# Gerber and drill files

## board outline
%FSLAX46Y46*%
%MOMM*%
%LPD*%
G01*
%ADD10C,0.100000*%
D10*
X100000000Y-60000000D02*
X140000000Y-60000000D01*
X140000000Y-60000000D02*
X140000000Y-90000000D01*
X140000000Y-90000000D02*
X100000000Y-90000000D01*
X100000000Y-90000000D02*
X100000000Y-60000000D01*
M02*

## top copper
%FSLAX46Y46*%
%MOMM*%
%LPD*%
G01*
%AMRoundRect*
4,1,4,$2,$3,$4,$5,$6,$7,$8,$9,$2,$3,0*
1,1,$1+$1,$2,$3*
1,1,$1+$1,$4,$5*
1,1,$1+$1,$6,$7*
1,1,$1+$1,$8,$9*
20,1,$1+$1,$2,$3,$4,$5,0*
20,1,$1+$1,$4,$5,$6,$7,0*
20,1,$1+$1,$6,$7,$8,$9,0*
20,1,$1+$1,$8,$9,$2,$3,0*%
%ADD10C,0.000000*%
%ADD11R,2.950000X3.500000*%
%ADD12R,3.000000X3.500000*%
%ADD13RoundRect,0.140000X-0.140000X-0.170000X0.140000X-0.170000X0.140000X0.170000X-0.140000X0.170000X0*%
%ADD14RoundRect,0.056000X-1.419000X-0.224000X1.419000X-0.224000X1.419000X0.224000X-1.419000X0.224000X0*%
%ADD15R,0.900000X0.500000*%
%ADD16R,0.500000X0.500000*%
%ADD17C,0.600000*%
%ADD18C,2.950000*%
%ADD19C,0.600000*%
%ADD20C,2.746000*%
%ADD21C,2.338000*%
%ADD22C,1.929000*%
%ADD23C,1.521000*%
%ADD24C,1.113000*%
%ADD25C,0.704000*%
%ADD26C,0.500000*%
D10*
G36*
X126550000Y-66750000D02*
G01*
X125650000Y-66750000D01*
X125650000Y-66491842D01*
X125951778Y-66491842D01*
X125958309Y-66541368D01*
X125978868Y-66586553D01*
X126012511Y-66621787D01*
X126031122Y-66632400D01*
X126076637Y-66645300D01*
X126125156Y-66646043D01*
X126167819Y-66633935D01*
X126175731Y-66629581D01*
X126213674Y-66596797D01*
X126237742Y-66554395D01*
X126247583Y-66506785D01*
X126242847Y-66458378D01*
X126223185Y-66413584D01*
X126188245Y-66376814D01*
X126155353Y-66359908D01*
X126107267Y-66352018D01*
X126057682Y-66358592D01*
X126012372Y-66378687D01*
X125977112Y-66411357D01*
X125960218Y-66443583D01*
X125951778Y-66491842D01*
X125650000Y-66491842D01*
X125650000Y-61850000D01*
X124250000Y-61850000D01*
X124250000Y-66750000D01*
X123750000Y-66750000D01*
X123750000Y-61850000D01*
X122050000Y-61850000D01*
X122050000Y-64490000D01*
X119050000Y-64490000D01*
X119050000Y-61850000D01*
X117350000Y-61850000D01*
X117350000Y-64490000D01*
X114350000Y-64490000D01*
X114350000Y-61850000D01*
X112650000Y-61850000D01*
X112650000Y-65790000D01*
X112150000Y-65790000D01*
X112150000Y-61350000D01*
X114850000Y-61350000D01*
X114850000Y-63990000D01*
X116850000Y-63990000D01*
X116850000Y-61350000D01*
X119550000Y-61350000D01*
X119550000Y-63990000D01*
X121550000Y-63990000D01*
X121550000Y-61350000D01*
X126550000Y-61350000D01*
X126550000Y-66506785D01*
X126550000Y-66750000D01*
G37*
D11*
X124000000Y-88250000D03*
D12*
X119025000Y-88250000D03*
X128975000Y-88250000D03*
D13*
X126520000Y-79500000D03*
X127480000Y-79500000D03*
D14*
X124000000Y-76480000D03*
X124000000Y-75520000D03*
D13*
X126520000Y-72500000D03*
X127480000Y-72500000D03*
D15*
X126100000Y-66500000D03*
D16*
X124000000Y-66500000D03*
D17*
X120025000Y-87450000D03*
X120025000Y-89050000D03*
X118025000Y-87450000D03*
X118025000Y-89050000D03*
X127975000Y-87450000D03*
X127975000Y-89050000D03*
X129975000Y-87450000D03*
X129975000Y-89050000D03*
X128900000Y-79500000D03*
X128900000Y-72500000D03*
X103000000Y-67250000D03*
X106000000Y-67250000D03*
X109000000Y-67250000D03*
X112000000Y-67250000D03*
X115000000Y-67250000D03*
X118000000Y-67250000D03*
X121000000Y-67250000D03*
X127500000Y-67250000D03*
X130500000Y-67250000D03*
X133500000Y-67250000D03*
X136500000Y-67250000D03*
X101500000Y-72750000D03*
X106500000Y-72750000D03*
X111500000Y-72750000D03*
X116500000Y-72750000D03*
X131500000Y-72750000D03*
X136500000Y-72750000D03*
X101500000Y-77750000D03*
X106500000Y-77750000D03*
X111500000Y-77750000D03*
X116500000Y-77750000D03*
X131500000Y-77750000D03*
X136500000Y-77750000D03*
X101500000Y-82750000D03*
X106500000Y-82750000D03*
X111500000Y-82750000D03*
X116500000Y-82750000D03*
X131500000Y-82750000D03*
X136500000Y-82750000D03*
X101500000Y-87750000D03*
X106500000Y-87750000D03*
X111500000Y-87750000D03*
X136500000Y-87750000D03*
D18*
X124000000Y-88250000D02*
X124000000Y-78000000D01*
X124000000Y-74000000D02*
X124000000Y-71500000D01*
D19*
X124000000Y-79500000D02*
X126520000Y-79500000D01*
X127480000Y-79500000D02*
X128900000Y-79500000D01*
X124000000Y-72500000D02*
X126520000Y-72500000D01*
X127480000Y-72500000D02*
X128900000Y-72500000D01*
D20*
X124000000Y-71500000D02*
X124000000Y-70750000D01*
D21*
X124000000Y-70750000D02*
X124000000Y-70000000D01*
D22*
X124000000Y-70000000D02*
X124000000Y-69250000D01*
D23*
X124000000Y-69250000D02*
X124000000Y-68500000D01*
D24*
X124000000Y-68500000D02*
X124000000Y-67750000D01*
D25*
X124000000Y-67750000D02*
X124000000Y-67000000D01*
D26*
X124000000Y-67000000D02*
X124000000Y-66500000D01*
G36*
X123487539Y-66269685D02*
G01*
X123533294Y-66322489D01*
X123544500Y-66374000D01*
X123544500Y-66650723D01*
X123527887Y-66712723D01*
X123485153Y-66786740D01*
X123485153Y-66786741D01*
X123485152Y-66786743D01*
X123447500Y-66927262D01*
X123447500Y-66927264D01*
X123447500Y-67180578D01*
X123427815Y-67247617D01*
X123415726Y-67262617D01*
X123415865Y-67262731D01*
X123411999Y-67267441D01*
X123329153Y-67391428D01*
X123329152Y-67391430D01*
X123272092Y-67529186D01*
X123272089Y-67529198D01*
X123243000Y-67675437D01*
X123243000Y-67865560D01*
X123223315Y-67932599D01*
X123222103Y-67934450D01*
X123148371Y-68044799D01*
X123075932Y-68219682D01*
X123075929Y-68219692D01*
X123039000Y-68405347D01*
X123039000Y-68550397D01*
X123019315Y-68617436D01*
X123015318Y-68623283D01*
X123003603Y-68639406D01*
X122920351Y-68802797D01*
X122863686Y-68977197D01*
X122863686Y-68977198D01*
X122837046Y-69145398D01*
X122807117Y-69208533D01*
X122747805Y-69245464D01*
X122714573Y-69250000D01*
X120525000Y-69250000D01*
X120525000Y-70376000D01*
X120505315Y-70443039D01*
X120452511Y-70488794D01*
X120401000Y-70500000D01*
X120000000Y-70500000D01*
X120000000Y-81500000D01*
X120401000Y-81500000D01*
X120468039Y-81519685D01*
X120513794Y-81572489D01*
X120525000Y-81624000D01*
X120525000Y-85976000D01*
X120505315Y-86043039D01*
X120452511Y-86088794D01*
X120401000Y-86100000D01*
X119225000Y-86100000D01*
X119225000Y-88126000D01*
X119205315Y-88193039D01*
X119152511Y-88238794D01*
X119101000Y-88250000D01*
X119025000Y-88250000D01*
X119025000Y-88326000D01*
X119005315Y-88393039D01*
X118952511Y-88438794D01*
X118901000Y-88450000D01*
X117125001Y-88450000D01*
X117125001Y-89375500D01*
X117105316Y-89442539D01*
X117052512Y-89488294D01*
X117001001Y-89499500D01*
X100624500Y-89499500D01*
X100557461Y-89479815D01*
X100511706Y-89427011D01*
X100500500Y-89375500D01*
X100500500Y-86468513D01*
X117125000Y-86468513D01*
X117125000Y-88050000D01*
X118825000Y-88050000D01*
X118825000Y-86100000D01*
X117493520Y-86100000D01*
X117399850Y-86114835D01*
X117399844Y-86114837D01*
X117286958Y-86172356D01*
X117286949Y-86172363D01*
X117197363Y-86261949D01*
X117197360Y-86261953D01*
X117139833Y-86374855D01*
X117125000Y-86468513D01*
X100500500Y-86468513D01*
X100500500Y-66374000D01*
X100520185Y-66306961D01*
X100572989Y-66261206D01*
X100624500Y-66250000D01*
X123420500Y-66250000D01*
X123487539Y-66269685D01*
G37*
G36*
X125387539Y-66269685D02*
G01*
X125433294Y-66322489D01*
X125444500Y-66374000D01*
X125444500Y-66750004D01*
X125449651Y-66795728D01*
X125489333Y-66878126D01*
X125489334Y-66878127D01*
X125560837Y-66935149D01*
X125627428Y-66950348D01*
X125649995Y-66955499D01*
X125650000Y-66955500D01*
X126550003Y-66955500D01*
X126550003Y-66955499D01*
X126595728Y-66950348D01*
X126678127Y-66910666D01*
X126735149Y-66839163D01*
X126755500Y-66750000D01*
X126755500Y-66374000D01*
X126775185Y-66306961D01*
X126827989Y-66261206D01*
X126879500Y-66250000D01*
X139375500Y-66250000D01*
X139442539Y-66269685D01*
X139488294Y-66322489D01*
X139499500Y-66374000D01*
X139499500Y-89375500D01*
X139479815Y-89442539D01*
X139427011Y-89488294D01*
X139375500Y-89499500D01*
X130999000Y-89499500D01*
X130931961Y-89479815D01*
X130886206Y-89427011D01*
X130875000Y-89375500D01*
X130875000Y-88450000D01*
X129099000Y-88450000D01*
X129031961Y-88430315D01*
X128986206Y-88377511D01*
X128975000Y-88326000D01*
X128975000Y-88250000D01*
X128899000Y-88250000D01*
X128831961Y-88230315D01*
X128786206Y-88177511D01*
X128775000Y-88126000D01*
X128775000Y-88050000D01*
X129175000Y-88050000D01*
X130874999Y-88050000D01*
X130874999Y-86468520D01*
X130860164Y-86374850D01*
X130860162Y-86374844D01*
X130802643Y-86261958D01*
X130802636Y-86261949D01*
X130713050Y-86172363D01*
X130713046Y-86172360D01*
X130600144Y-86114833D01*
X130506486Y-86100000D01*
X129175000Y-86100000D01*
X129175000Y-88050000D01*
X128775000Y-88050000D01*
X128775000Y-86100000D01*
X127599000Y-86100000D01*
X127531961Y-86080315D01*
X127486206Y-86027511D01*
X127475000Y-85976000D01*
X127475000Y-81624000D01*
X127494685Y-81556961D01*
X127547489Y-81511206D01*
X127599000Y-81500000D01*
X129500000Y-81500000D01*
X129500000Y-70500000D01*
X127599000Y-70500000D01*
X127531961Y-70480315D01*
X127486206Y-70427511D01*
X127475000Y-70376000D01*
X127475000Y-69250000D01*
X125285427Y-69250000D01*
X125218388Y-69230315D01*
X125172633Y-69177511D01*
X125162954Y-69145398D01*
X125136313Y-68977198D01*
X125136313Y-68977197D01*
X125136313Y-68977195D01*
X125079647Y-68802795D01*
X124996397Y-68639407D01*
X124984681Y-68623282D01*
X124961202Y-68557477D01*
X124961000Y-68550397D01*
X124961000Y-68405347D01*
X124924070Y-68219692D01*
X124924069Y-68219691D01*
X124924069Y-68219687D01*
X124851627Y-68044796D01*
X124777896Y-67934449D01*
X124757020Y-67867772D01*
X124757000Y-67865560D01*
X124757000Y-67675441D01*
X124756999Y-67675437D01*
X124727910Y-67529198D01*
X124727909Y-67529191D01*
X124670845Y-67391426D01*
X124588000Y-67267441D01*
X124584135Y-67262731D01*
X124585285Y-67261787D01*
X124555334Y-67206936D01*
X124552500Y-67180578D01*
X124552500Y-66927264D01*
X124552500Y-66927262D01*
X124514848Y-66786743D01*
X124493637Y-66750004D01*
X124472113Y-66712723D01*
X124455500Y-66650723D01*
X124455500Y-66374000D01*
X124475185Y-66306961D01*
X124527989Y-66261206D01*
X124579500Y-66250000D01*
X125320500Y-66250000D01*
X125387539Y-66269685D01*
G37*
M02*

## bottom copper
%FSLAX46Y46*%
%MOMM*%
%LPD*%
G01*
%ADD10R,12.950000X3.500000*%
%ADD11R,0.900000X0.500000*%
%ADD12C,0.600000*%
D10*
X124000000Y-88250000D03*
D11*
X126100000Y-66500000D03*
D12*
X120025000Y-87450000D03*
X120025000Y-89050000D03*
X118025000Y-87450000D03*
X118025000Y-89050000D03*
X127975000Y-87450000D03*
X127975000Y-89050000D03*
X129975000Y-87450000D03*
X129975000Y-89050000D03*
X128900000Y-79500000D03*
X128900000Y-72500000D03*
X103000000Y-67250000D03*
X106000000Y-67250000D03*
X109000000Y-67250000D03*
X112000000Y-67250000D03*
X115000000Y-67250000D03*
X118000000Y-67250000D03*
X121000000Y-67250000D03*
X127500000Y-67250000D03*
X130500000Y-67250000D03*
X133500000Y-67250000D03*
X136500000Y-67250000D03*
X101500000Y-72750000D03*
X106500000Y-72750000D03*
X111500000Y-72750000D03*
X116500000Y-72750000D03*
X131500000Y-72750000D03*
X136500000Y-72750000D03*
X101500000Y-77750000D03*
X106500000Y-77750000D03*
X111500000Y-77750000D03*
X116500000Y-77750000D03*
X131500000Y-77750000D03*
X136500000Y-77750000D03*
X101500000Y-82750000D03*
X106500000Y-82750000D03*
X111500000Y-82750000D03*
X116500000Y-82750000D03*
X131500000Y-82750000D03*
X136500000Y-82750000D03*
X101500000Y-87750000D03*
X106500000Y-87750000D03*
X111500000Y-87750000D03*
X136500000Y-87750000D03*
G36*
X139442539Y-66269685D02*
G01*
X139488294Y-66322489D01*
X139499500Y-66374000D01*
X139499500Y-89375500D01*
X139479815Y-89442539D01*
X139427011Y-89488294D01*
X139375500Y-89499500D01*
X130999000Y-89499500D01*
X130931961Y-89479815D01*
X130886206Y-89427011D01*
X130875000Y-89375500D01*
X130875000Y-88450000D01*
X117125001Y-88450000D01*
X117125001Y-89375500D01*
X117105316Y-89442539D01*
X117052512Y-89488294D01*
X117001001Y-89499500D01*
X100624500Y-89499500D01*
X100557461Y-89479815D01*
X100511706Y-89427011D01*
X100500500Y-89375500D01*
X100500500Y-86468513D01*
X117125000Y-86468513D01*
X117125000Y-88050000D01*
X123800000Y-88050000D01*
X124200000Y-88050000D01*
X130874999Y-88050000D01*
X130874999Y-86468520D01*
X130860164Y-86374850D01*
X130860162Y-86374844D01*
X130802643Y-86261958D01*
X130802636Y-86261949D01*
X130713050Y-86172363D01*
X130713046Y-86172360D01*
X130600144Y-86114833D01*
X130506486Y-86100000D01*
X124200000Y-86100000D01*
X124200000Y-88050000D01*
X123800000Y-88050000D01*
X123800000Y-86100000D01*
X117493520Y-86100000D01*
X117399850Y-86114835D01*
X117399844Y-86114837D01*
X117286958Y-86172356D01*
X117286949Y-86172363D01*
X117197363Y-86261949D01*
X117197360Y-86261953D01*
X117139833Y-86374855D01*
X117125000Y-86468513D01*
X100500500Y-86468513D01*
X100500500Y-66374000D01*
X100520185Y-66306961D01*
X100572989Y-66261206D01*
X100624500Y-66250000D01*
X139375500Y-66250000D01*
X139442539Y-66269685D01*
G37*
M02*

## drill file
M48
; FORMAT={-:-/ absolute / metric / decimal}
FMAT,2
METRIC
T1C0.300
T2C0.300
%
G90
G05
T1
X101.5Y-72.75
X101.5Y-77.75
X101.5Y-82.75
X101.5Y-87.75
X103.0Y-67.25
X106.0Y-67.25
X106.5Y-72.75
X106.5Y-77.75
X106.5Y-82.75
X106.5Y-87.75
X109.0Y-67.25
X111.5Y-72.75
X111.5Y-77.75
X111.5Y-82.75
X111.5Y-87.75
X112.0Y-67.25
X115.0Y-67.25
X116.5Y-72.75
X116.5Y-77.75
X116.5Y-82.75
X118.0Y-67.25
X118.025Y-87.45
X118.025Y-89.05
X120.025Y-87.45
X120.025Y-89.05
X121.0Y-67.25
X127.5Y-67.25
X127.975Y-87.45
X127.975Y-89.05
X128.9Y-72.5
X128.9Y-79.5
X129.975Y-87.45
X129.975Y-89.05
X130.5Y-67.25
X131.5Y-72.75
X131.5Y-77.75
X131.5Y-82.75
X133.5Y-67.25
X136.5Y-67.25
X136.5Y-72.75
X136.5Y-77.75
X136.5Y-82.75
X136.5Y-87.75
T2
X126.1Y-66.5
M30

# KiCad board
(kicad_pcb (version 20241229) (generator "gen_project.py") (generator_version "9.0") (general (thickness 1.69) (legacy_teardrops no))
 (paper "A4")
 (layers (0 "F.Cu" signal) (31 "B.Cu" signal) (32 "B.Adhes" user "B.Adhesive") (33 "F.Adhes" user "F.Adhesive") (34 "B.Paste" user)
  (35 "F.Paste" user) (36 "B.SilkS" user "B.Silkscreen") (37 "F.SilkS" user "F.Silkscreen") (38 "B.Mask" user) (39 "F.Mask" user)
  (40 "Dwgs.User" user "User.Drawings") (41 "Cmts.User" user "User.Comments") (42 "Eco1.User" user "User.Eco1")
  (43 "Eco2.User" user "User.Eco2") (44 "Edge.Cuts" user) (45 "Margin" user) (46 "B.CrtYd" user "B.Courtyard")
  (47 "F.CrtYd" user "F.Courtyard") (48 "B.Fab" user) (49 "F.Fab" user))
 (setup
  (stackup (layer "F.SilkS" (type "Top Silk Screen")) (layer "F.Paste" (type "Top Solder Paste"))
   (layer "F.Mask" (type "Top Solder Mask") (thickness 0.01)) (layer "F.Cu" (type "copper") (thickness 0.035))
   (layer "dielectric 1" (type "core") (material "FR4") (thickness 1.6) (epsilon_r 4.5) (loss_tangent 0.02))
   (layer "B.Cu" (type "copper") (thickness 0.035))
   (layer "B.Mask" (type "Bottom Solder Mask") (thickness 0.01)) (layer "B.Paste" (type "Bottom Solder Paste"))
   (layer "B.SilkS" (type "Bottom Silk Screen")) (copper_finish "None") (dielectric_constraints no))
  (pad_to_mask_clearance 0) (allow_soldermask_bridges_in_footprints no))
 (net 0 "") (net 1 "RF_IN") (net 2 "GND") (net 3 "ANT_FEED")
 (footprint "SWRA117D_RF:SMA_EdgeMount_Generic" (layer "F.Cu") (at 124 90 90)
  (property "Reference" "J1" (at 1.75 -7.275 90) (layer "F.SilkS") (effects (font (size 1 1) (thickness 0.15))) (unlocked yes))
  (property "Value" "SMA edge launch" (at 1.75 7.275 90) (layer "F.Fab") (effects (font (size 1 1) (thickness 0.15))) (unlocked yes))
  (pad "1" smd rect (at 1.75 0 90) (size 3.5 2.95) (layers "F.Cu" "F.Paste" "F.Mask") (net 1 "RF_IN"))
  (pad "2" smd rect (at 1.75 -4.975 90) (size 3.5 3) (layers "F.Cu" "F.Paste" "F.Mask") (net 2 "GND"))
  (pad "2" smd rect (at 1.75 4.975 90) (size 3.5 3) (layers "F.Cu" "F.Paste" "F.Mask") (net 2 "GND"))
  (pad "2" smd rect (at 1.75 0 90) (size 3.5 12.95) (layers "B.Cu" "B.Paste" "B.Mask") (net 2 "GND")))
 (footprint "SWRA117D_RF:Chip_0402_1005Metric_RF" (layer "F.Cu") (at 127 79.5)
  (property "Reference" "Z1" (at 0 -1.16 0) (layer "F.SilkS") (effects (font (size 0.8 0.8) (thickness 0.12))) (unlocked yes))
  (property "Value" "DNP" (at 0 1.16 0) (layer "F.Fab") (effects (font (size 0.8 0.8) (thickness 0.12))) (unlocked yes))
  (pad "1" smd roundrect (at -0.48 0) (size 0.56 0.62) (layers "F.Cu" "F.Paste" "F.Mask") (roundrect_rratio 0.25) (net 1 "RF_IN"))
  (pad "2" smd roundrect (at 0.48 0) (size 0.56 0.62) (layers "F.Cu" "F.Paste" "F.Mask") (roundrect_rratio 0.25) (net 2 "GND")))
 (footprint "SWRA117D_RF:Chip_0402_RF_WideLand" (layer "F.Cu") (at 124 76)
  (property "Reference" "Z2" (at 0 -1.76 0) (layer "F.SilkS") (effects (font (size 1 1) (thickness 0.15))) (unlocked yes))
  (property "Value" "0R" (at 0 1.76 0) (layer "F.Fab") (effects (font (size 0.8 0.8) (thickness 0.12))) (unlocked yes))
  (pad "1" smd roundrect (at 0 0.48) (size 2.95 0.56) (layers "F.Cu" "F.Paste" "F.Mask") (roundrect_rratio 0.1) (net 1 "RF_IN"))
  (pad "2" smd roundrect (at 0 -0.48) (size 2.95 0.56) (layers "F.Cu" "F.Paste" "F.Mask") (roundrect_rratio 0.1) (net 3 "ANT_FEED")))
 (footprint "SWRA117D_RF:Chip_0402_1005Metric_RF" (layer "F.Cu") (at 127 72.5)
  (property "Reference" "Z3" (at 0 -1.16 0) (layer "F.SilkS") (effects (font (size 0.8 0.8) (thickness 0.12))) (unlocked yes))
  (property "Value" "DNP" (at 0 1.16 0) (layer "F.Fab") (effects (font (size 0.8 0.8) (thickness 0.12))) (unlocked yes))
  (pad "1" smd roundrect (at -0.48 0) (size 0.56 0.62) (layers "F.Cu" "F.Paste" "F.Mask") (roundrect_rratio 0.25) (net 3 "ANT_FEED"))
  (pad "2" smd roundrect (at 0.48 0) (size 0.56 0.62) (layers "F.Cu" "F.Paste" "F.Mask") (roundrect_rratio 0.25) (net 2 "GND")))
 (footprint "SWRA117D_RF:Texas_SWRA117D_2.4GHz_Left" (layer "F.Cu") (at 124 66.5)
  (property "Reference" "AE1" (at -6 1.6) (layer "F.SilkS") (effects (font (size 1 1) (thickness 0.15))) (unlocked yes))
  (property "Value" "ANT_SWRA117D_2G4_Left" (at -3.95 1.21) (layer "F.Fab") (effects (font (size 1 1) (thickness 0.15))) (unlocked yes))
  (fp_poly
   (pts (xy -2.45 -2.51) (xy -4.45 -2.51) (xy -4.45 -5.15) (xy -7.15 -5.15) (xy -7.15 -2.51) (xy -9.15 -2.51) (xy -9.15 -5.15)
    (xy -11.85 -5.15) (xy -11.85 -0.71) (xy -11.35 -0.71) (xy -11.35 -4.65) (xy -9.65 -4.65) (xy -9.65 -2.01) (xy -6.65 -2.01)
    (xy -6.65 -4.65) (xy -4.95 -4.65) (xy -4.95 -2.01) (xy -1.95 -2.01) (xy -1.95 -4.65) (xy -0.25 -4.65) (xy -0.25 0.25) (xy 0.25 0.25)
    (xy 0.25 -4.65) (xy 1.65 -4.65) (xy 1.65 0.25) (xy 2.55 0.25) (xy 2.55 0.006785) (xy 2.247583 0.006785) (xy 2.237742 0.054395)
    (xy 2.213674 0.096797) (xy 2.175731 0.129581) (xy 2.167819 0.133935) (xy 2.125156 0.146043) (xy 2.076637 0.1453) (xy 2.031122 0.1324)
    (xy 2.012511 0.121787) (xy 1.978868 0.086553) (xy 1.958309 0.041368) (xy 1.951778 -0.008158) (xy 1.960218 -0.056417)
    (xy 1.977112 -0.088643) (xy 2.012372 -0.121313) (xy 2.057682 -0.141408) (xy 2.107267 -0.147982) (xy 2.155353 -0.140092)
    (xy 2.188245 -0.123186) (xy 2.223185 -0.086416) (xy 2.242847 -0.041622) (xy 2.247583 0.006785) (xy 2.55 0.006785) (xy 2.55 -5.15)
    (xy -2.45 -5.15) (xy -2.45 -2.51))
   (stroke (width 0) (type solid)) (fill yes) (layer "F.Cu"))
  (pad "2" thru_hole rect (at 2.1 0) (size 0.9 0.5) (drill 0.3) (layers "*.Cu") (zone_connect 2) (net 2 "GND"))
  (pad "1" smd rect (at 0 0) (size 0.5 0.5) (layers "F.Cu") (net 3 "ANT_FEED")))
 (gr_line (start 100 60) (end 140 60) (stroke (width 0.1) (type solid)) (layer "Edge.Cuts"))
 (gr_line (start 140 60) (end 140 90) (stroke (width 0.1) (type solid)) (layer "Edge.Cuts"))
 (gr_line (start 140 90) (end 100 90) (stroke (width 0.1) (type solid)) (layer "Edge.Cuts"))
 (gr_line (start 100 90) (end 100 60) (stroke (width 0.1) (type solid)) (layer "Edge.Cuts"))
 (segment (start 124 88.25) (end 124 78) (width 2.95) (layer "F.Cu") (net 1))
 (segment (start 124 74) (end 124 71.5) (width 2.95) (layer "F.Cu") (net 3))
 (segment (start 124 79.5) (end 126.52 79.5) (width 0.6) (layer "F.Cu") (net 1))
 (segment (start 127.48 79.5) (end 128.9 79.5) (width 0.6) (layer "F.Cu") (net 2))
 (segment (start 124 72.5) (end 126.52 72.5) (width 0.6) (layer "F.Cu") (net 3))
 (segment (start 127.48 72.5) (end 128.9 72.5) (width 0.6) (layer "F.Cu") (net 2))
 (segment (start 124 71.5) (end 124 70.75) (width 2.746) (layer "F.Cu") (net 3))
 (segment (start 124 70.75) (end 124 70) (width 2.338) (layer "F.Cu") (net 3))
 (segment (start 124 70) (end 124 69.25) (width 1.929) (layer "F.Cu") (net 3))
 (segment (start 124 69.25) (end 124 68.5) (width 1.521) (layer "F.Cu") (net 3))
 (segment (start 124 68.5) (end 124 67.75) (width 1.113) (layer "F.Cu") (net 3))
 (segment (start 124 67.75) (end 124 67) (width 0.704) (layer "F.Cu") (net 3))
 (segment (start 124 67) (end 124 66.5) (width 0.5) (layer "F.Cu") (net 3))
 (via (at 120.025 87.45) (size 0.6) (drill 0.3) (layers "F.Cu" "B.Cu") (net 2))
 (via (at 120.025 89.05) (size 0.6) (drill 0.3) (layers "F.Cu" "B.Cu") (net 2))
 (via (at 118.025 87.45) (size 0.6) (drill 0.3) (layers "F.Cu" "B.Cu") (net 2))
 (via (at 118.025 89.05) (size 0.6) (drill 0.3) (layers "F.Cu" "B.Cu") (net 2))
 (via (at 127.975 87.45) (size 0.6) (drill 0.3) (layers "F.Cu" "B.Cu") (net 2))
 (via (at 127.975 89.05) (size 0.6) (drill 0.3) (layers "F.Cu" "B.Cu") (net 2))
 (via (at 129.975 87.45) (size 0.6) (drill 0.3) (layers "F.Cu" "B.Cu") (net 2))
 (via (at 129.975 89.05) (size 0.6) (drill 0.3) (layers "F.Cu" "B.Cu") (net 2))
 (via (at 128.9 79.5) (size 0.6) (drill 0.3) (layers "F.Cu" "B.Cu") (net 2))
 (via (at 128.9 72.5) (size 0.6) (drill 0.3) (layers "F.Cu" "B.Cu") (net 2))
 (via (at 103 67.25) (size 0.6) (drill 0.3) (layers "F.Cu" "B.Cu") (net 2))
 (via (at 106 67.25) (size 0.6) (drill 0.3) (layers "F.Cu" "B.Cu") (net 2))
 (via (at 109 67.25) (size 0.6) (drill 0.3) (layers "F.Cu" "B.Cu") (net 2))
 (via (at 112 67.25) (size 0.6) (drill 0.3) (layers "F.Cu" "B.Cu") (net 2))
 (via (at 115 67.25) (size 0.6) (drill 0.3) (layers "F.Cu" "B.Cu") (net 2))
 (via (at 118 67.25) (size 0.6) (drill 0.3) (layers "F.Cu" "B.Cu") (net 2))
 (via (at 121 67.25) (size 0.6) (drill 0.3) (layers "F.Cu" "B.Cu") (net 2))
 (via (at 127.5 67.25) (size 0.6) (drill 0.3) (layers "F.Cu" "B.Cu") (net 2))
 (via (at 130.5 67.25) (size 0.6) (drill 0.3) (layers "F.Cu" "B.Cu") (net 2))
 (via (at 133.5 67.25) (size 0.6) (drill 0.3) (layers "F.Cu" "B.Cu") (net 2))
 (via (at 136.5 67.25) (size 0.6) (drill 0.3) (layers "F.Cu" "B.Cu") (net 2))
 (via (at 101.5 72.75) (size 0.6) (drill 0.3) (layers "F.Cu" "B.Cu") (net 2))
 (via (at 106.5 72.75) (size 0.6) (drill 0.3) (layers "F.Cu" "B.Cu") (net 2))
 (via (at 111.5 72.75) (size 0.6) (drill 0.3) (layers "F.Cu" "B.Cu") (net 2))
 (via (at 116.5 72.75) (size 0.6) (drill 0.3) (layers "F.Cu" "B.Cu") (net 2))
 (via (at 131.5 72.75) (size 0.6) (drill 0.3) (layers "F.Cu" "B.Cu") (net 2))
 (via (at 136.5 72.75) (size 0.6) (drill 0.3) (layers "F.Cu" "B.Cu") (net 2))
 (via (at 101.5 77.75) (size 0.6) (drill 0.3) (layers "F.Cu" "B.Cu") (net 2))
 (via (at 106.5 77.75) (size 0.6) (drill 0.3) (layers "F.Cu" "B.Cu") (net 2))
 (via (at 111.5 77.75) (size 0.6) (drill 0.3) (layers "F.Cu" "B.Cu") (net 2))
 (via (at 116.5 77.75) (size 0.6) (drill 0.3) (layers "F.Cu" "B.Cu") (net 2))
 (via (at 131.5 77.75) (size 0.6) (drill 0.3) (layers "F.Cu" "B.Cu") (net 2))
 (via (at 136.5 77.75) (size 0.6) (drill 0.3) (layers "F.Cu" "B.Cu") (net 2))
 (via (at 101.5 82.75) (size 0.6) (drill 0.3) (layers "F.Cu" "B.Cu") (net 2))
 (via (at 106.5 82.75) (size 0.6) (drill 0.3) (layers "F.Cu" "B.Cu") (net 2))
 (via (at 111.5 82.75) (size 0.6) (drill 0.3) (layers "F.Cu" "B.Cu") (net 2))
 (via (at 116.5 82.75) (size 0.6) (drill 0.3) (layers "F.Cu" "B.Cu") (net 2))
 (via (at 131.5 82.75) (size 0.6) (drill 0.3) (layers "F.Cu" "B.Cu") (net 2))
 (via (at 136.5 82.75) (size 0.6) (drill 0.3) (layers "F.Cu" "B.Cu") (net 2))
 (via (at 101.5 87.75) (size 0.6) (drill 0.3) (layers "F.Cu" "B.Cu") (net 2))
 (via (at 106.5 87.75) (size 0.6) (drill 0.3) (layers "F.Cu" "B.Cu") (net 2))
 (via (at 111.5 87.75) (size 0.6) (drill 0.3) (layers "F.Cu" "B.Cu") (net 2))
 (via (at 136.5 87.75) (size 0.6) (drill 0.3) (layers "F.Cu" "B.Cu") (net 2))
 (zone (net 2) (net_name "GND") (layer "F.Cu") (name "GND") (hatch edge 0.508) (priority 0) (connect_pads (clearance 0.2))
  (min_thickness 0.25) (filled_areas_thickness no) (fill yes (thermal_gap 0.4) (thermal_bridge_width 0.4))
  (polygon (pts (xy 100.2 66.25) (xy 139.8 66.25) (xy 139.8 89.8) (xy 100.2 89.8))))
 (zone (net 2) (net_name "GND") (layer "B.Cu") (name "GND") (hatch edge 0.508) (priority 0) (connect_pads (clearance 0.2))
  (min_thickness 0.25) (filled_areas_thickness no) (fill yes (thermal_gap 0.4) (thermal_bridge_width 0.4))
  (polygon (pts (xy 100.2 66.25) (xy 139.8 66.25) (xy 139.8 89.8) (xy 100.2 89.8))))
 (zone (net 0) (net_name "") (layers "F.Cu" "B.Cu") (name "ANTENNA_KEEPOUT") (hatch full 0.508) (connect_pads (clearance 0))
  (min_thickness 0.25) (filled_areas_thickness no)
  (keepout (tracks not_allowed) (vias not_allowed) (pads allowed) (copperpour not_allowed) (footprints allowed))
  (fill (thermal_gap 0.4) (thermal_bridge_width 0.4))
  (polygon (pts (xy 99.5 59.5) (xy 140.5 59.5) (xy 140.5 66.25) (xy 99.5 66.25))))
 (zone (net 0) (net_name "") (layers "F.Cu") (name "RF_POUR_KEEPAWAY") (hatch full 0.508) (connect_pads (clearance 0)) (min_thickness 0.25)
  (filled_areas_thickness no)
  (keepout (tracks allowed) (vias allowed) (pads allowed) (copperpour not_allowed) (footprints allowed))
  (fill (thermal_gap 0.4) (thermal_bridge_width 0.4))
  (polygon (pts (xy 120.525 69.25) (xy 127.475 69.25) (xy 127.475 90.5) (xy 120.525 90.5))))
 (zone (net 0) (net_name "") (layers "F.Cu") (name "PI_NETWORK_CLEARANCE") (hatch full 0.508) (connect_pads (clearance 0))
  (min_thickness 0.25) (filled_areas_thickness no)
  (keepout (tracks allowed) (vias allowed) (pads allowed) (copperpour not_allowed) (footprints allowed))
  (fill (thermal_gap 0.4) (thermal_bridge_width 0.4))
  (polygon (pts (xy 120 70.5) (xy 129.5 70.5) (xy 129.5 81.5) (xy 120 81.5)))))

